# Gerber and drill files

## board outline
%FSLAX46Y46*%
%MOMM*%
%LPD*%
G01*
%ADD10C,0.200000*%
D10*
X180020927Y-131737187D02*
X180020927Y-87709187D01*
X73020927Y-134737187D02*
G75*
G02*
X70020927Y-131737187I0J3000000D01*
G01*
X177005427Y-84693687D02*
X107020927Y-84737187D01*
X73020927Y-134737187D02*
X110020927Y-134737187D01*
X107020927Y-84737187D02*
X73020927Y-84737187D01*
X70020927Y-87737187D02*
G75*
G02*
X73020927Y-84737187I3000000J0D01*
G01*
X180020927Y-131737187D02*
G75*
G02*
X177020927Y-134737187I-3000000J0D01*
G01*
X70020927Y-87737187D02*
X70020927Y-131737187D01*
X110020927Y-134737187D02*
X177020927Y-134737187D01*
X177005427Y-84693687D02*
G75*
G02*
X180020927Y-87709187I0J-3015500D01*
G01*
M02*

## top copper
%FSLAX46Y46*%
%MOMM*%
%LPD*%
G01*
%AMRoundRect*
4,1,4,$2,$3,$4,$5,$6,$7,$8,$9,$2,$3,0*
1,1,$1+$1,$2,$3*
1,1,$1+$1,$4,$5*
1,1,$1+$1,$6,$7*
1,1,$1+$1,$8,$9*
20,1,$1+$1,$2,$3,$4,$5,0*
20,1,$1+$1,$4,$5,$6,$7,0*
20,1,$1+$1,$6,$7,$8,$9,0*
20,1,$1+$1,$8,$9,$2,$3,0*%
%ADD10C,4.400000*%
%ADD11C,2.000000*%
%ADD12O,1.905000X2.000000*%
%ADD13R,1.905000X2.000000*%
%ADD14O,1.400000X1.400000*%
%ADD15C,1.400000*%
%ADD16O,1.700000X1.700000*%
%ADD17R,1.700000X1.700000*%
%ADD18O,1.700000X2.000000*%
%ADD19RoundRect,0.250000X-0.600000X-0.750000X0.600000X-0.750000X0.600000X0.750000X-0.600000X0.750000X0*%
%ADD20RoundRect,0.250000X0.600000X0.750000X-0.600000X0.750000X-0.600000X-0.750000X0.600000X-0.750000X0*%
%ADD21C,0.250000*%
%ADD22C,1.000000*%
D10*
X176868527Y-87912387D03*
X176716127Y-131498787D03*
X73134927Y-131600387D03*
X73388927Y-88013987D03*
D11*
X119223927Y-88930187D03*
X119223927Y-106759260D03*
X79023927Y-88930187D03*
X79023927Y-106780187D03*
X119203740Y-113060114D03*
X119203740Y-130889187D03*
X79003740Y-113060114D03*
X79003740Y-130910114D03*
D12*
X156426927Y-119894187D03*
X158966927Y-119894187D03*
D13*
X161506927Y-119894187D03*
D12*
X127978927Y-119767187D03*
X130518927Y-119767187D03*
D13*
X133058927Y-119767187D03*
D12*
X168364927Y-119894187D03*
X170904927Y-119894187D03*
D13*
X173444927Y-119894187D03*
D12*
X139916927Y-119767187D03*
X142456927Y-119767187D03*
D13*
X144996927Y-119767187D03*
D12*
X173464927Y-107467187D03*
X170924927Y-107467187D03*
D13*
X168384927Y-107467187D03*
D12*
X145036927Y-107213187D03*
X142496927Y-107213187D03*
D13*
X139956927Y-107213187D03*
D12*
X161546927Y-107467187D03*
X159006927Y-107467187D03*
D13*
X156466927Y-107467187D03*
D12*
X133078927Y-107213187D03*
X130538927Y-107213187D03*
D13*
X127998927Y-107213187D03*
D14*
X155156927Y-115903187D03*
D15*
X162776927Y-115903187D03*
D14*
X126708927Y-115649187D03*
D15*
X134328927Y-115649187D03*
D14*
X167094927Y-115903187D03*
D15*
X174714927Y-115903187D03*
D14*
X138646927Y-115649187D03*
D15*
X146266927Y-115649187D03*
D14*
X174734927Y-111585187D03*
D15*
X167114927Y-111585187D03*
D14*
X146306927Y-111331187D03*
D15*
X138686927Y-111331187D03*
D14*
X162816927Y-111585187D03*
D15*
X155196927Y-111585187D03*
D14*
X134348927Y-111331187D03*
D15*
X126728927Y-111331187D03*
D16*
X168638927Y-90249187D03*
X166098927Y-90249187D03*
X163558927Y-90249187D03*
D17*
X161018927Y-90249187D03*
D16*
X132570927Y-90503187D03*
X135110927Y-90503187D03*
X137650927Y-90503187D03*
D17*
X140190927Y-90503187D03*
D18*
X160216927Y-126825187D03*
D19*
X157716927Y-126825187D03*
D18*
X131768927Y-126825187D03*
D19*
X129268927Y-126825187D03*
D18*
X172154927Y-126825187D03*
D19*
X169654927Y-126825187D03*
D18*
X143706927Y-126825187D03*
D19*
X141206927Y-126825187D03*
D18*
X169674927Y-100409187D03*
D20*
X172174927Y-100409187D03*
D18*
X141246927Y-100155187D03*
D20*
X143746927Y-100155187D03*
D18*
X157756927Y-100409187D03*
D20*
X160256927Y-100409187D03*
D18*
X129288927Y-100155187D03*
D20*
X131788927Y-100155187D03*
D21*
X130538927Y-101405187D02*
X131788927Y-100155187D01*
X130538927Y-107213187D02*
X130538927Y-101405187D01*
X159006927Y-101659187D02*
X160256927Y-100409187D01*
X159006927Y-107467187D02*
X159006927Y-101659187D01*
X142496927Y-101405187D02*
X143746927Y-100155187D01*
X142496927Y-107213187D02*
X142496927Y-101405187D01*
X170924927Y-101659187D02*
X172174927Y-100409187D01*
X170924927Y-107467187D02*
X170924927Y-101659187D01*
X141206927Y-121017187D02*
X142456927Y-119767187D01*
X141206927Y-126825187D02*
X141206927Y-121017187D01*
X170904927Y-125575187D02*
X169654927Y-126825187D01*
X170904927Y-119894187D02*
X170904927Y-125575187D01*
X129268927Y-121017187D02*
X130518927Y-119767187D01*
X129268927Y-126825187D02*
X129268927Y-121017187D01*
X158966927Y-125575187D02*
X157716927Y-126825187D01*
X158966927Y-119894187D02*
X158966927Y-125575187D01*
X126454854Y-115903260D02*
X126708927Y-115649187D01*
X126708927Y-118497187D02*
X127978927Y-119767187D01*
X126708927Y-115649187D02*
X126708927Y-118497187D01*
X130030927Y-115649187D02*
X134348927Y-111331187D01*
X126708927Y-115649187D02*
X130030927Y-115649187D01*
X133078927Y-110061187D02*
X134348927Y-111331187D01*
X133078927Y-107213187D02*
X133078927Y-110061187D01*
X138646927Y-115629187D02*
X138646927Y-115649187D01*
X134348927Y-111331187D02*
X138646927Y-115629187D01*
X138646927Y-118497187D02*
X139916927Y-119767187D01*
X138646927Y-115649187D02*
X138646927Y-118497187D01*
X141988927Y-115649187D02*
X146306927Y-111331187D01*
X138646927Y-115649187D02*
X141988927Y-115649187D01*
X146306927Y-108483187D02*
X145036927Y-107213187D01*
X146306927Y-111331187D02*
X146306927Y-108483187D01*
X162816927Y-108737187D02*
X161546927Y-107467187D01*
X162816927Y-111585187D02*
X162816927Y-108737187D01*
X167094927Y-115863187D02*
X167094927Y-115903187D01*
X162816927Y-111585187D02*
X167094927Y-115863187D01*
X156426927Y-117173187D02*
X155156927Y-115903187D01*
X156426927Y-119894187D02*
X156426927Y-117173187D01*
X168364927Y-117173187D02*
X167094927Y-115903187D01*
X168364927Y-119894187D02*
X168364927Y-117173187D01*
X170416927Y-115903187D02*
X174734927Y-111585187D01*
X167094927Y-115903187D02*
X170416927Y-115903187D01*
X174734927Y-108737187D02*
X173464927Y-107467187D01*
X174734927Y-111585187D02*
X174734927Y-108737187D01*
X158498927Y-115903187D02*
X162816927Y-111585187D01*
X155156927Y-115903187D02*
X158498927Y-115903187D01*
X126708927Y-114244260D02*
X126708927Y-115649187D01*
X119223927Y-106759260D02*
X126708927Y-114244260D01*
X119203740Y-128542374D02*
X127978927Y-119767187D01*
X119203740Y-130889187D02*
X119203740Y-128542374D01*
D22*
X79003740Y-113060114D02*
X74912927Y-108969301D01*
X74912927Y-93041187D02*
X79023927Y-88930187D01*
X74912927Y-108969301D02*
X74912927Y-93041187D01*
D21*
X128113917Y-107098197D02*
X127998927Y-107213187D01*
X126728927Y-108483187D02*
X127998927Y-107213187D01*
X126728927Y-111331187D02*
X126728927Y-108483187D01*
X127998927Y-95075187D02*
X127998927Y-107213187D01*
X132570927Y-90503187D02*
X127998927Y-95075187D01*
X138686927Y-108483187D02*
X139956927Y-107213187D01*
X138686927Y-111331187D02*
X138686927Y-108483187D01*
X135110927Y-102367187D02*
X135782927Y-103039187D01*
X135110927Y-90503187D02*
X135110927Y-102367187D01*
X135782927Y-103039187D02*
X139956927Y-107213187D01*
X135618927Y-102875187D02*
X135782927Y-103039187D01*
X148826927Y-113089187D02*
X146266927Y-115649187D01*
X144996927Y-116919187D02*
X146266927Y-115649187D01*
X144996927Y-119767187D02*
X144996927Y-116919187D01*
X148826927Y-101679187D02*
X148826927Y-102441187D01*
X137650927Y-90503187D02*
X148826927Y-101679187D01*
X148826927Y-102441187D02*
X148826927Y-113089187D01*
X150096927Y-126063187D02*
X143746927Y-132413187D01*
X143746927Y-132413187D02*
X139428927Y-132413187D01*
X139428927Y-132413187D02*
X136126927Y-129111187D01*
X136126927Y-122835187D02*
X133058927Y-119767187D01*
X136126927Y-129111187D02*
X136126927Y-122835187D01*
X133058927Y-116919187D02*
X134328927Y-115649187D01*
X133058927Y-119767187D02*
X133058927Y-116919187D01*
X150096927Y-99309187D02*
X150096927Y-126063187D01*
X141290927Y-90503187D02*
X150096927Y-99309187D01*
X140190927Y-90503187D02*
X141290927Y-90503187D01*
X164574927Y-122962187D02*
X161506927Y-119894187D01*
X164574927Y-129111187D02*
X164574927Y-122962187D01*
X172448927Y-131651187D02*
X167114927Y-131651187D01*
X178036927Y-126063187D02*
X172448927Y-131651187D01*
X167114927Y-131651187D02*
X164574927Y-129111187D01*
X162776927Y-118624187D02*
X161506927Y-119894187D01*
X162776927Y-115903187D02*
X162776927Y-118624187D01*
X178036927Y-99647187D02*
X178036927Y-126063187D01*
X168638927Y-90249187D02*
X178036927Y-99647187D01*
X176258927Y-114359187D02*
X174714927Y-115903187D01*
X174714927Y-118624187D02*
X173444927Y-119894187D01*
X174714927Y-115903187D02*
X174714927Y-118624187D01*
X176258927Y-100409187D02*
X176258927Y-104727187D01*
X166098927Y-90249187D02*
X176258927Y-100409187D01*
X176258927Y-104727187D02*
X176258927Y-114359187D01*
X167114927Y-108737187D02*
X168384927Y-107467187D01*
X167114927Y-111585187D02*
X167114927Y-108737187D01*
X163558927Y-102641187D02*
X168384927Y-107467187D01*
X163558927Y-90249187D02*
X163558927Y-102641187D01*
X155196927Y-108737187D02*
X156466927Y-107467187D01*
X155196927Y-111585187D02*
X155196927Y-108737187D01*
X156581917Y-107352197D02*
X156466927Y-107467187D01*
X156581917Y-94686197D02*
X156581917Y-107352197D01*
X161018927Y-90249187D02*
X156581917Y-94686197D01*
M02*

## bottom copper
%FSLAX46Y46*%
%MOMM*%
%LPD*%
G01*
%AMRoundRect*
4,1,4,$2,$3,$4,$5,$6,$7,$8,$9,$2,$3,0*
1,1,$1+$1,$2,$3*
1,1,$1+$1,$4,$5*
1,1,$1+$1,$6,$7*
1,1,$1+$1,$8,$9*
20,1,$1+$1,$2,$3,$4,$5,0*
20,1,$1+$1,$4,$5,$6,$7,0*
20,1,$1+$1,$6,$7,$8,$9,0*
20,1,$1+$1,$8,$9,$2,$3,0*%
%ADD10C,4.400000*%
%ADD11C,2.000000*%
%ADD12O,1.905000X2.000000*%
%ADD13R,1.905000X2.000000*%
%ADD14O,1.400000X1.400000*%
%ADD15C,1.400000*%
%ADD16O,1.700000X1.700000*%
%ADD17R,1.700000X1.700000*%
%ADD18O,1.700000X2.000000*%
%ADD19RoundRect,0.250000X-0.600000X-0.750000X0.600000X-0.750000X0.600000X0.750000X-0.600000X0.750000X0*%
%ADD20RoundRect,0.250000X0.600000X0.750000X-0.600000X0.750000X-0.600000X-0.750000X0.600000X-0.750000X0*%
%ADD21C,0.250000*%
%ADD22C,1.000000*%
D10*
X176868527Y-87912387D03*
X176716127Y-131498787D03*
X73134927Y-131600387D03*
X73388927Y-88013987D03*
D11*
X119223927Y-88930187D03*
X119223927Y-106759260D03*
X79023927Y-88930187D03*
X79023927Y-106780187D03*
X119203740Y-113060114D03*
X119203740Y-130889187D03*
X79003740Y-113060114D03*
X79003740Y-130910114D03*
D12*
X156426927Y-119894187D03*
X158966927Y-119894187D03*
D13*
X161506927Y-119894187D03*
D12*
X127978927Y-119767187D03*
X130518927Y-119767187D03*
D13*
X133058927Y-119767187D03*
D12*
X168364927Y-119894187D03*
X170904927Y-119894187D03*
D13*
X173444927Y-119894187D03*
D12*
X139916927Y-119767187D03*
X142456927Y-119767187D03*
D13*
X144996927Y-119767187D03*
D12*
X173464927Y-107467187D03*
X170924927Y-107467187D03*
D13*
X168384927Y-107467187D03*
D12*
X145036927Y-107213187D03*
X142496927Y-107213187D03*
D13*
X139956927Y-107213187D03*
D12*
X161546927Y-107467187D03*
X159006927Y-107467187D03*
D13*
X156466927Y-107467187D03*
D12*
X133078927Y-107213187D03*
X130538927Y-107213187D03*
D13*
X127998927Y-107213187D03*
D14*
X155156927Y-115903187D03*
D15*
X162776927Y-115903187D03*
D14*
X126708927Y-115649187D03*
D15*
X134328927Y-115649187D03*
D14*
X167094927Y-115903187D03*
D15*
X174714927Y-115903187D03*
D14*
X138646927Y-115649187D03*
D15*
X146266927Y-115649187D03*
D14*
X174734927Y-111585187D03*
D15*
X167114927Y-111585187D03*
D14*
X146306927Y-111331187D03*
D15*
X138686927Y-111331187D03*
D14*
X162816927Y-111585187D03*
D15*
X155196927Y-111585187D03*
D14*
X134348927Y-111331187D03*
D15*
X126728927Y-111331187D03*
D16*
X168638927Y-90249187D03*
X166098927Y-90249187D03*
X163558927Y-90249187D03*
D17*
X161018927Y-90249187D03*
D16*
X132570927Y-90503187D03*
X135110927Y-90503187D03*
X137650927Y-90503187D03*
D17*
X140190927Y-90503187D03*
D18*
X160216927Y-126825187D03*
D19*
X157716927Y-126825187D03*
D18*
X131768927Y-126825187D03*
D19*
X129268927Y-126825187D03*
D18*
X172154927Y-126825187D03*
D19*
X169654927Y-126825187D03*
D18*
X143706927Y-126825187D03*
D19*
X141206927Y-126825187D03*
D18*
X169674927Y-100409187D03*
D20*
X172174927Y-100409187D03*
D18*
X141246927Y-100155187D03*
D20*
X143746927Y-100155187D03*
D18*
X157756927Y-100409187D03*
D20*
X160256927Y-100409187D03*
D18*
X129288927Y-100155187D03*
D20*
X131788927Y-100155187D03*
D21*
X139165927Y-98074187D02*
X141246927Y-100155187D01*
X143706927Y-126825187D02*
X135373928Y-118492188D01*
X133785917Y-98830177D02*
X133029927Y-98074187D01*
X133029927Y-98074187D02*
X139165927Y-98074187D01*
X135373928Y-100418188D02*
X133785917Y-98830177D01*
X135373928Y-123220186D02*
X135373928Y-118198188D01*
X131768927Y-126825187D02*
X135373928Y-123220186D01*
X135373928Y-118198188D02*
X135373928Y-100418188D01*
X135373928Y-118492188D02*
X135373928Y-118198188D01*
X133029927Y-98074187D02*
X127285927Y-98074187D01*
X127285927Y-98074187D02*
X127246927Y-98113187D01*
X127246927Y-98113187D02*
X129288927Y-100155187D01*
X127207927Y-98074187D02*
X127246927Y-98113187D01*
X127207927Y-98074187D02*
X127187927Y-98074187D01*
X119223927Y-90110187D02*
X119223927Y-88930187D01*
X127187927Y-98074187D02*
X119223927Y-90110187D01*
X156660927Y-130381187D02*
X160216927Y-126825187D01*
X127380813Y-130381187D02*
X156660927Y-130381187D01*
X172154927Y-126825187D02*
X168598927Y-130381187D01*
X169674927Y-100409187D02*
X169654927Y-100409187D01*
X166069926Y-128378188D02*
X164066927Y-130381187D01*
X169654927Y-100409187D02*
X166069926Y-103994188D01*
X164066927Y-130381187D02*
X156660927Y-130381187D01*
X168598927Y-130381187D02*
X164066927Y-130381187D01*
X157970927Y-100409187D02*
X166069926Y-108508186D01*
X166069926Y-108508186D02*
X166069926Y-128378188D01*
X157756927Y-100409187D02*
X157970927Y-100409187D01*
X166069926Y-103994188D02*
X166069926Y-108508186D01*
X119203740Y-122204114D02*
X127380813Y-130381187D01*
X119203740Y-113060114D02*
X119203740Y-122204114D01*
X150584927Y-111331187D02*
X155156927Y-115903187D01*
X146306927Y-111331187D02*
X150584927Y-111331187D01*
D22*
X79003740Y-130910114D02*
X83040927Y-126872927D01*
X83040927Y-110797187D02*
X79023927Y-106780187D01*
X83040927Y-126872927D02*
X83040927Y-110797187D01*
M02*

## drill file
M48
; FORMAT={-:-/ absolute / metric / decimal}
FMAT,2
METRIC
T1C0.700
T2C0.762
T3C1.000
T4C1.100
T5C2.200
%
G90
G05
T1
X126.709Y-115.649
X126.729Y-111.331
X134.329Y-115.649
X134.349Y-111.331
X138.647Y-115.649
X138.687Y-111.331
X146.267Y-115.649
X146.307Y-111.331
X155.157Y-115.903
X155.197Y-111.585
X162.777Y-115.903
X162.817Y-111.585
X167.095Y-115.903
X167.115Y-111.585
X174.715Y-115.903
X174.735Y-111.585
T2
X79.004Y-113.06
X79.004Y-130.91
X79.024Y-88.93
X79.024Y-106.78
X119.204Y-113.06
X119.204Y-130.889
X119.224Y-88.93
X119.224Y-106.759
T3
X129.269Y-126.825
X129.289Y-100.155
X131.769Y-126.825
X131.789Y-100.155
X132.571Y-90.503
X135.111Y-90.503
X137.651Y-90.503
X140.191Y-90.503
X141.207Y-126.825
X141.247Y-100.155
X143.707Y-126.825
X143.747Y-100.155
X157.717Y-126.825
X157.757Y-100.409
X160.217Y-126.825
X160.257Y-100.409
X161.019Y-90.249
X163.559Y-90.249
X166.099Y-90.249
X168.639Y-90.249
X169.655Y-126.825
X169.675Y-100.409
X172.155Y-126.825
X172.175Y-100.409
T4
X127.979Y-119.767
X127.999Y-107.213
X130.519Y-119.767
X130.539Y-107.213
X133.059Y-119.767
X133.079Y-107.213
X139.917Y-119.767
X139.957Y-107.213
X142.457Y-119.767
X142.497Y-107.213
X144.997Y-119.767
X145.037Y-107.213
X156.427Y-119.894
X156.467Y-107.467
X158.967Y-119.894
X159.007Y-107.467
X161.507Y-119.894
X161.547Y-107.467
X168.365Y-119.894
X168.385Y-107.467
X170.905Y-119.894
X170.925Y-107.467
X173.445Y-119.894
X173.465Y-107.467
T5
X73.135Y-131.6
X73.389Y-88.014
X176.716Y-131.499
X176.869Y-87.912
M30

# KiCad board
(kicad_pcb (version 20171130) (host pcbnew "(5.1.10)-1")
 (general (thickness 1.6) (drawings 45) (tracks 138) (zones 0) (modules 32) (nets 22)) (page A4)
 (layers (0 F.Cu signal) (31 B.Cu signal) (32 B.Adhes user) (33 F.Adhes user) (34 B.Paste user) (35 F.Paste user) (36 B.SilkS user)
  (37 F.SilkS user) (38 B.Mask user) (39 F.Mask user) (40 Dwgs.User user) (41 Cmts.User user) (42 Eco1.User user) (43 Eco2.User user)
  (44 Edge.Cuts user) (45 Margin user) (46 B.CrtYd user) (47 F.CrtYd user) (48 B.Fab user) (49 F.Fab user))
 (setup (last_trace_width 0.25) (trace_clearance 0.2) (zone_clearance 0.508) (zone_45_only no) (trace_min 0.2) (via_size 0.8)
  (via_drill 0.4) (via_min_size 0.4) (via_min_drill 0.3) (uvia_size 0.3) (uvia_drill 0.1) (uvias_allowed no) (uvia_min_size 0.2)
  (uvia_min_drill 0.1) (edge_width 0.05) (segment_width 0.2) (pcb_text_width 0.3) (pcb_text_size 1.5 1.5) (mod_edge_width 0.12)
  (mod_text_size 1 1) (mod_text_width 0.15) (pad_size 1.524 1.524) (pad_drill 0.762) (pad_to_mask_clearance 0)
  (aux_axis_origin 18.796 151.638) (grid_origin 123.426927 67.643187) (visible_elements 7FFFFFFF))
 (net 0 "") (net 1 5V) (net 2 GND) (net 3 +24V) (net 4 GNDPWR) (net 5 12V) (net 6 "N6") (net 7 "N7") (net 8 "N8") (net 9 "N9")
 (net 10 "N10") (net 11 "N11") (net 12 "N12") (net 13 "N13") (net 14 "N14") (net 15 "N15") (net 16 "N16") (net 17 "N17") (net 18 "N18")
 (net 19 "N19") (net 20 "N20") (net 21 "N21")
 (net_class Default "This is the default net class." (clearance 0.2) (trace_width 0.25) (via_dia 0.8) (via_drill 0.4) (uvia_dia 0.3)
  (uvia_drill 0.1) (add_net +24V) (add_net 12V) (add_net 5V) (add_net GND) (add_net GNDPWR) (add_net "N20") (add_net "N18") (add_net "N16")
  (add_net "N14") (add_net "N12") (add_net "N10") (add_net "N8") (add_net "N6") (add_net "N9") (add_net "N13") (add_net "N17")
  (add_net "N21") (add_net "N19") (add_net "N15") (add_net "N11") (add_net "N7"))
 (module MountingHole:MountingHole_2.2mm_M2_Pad (layer F.Cu) (at 176.868527 87.912387)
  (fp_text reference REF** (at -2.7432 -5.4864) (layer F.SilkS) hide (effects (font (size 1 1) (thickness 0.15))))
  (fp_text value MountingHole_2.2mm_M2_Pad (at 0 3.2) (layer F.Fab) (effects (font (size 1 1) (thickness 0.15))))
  (pad 1 thru_hole circle (at 0 0) (size 4.4 4.4) (drill 2.2) (layers *.Cu *.Mask)))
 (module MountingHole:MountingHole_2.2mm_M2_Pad (layer F.Cu) (at 176.716127 131.498787)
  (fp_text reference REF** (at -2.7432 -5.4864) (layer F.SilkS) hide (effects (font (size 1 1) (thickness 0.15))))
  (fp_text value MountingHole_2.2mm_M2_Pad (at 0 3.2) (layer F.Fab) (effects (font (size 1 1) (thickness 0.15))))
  (pad 1 thru_hole circle (at 0 0) (size 4.4 4.4) (drill 2.2) (layers *.Cu *.Mask)))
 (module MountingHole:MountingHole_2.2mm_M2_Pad (layer F.Cu) (at 73.134927 131.600387)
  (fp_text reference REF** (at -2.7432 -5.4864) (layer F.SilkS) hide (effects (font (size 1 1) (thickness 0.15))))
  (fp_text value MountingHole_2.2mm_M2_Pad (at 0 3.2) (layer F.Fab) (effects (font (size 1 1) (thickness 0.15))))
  (pad 1 thru_hole circle (at 0 0) (size 4.4 4.4) (drill 2.2) (layers *.Cu *.Mask)))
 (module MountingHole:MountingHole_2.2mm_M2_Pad (layer F.Cu) (at 73.388927 88.013987)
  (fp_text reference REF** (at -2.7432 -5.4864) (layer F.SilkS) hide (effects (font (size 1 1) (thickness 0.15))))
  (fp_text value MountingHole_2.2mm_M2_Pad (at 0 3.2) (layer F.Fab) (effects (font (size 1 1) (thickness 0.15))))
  (pad 1 thru_hole circle (at 0 0) (size 4.4 4.4) (drill 2.2) (layers *.Cu *.Mask)))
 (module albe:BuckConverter (layer F.Cu) (at 99.825114 97.86926 270)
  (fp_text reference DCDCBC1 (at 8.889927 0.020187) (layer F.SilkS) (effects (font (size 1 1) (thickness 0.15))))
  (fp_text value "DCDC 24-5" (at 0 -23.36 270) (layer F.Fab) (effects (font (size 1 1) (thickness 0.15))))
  (pad 4 thru_hole circle (at -8.939073 -19.398813 270) (size 2 2) (drill 0.762) (layers *.Cu *.Mask) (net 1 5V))
  (pad 3 thru_hole circle (at 8.89 -19.398813 270) (size 2 2) (drill 0.762) (layers *.Cu *.Mask) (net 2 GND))
  (pad 2 thru_hole circle (at -8.939073 20.801187 270) (size 2 2) (drill 0.762) (layers *.Cu *.Mask) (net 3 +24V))
  (pad 1 thru_hole circle (at 8.910927 20.801187 270) (size 2 2) (drill 0.762) (layers *.Cu *.Mask) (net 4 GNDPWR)))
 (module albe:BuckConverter (layer F.Cu) (at 99.804927 121.999187 270)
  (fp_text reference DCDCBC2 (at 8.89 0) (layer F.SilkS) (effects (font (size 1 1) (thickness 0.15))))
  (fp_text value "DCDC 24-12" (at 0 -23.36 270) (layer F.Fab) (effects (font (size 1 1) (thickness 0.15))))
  (pad 4 thru_hole circle (at -8.939073 -19.398813 270) (size 2 2) (drill 0.762) (layers *.Cu *.Mask) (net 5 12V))
  (pad 3 thru_hole circle (at 8.89 -19.398813 270) (size 2 2) (drill 0.762) (layers *.Cu *.Mask) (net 2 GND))
  (pad 2 thru_hole circle (at -8.939073 20.801187 270) (size 2 2) (drill 0.762) (layers *.Cu *.Mask) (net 3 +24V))
  (pad 1 thru_hole circle (at 8.910927 20.801187 270) (size 2 2) (drill 0.762) (layers *.Cu *.Mask) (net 4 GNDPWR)))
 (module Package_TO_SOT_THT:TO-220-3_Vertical (layer F.Cu) (at 161.506927 119.894187 180)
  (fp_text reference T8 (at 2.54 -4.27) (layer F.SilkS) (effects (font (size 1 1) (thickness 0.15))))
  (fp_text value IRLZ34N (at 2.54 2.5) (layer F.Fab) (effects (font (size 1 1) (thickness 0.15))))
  (pad 3 thru_hole oval (at 5.08 0 180) (size 1.905 2) (drill 1.1) (layers *.Cu *.Mask) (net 2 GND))
  (pad 2 thru_hole oval (at 2.54 0 180) (size 1.905 2) (drill 1.1) (layers *.Cu *.Mask) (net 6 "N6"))
  (pad 1 thru_hole rect (at 0 0 180) (size 1.905 2) (drill 1.1) (layers *.Cu *.Mask) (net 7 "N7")))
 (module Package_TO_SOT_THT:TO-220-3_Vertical (layer F.Cu) (at 133.058927 119.767187 180)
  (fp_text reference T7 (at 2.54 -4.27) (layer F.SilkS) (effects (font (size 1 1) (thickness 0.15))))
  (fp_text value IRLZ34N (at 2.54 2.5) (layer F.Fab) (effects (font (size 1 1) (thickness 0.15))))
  (pad 3 thru_hole oval (at 5.08 0 180) (size 1.905 2) (drill 1.1) (layers *.Cu *.Mask) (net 2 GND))
  (pad 2 thru_hole oval (at 2.54 0 180) (size 1.905 2) (drill 1.1) (layers *.Cu *.Mask) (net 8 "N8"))
  (pad 1 thru_hole rect (at 0 0 180) (size 1.905 2) (drill 1.1) (layers *.Cu *.Mask) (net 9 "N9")))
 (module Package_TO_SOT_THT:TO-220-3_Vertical (layer F.Cu) (at 173.444927 119.894187 180)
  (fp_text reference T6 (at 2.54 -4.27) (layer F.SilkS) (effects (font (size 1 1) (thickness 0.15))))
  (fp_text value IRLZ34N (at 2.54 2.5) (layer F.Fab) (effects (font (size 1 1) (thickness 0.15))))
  (pad 3 thru_hole oval (at 5.08 0 180) (size 1.905 2) (drill 1.1) (layers *.Cu *.Mask) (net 2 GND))
  (pad 2 thru_hole oval (at 2.54 0 180) (size 1.905 2) (drill 1.1) (layers *.Cu *.Mask) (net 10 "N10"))
  (pad 1 thru_hole rect (at 0 0 180) (size 1.905 2) (drill 1.1) (layers *.Cu *.Mask) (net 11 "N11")))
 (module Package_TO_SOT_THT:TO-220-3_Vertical (layer F.Cu) (at 144.996927 119.767187 180)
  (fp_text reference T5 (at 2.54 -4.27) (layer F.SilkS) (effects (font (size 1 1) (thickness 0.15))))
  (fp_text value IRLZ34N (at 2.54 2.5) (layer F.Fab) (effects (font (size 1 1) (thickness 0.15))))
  (pad 3 thru_hole oval (at 5.08 0 180) (size 1.905 2) (drill 1.1) (layers *.Cu *.Mask) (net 2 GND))
  (pad 2 thru_hole oval (at 2.54 0 180) (size 1.905 2) (drill 1.1) (layers *.Cu *.Mask) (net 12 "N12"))
  (pad 1 thru_hole rect (at 0 0 180) (size 1.905 2) (drill 1.1) (layers *.Cu *.Mask) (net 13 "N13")))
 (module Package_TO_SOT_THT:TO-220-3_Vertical (layer F.Cu) (at 168.384927 107.467187)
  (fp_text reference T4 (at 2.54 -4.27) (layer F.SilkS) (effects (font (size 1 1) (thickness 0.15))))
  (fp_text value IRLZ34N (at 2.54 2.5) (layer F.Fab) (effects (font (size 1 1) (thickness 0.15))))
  (pad 3 thru_hole oval (at 5.08 0) (size 1.905 2) (drill 1.1) (layers *.Cu *.Mask) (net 2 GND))
  (pad 2 thru_hole oval (at 2.54 0) (size 1.905 2) (drill 1.1) (layers *.Cu *.Mask) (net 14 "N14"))
  (pad 1 thru_hole rect (at 0 0) (size 1.905 2) (drill 1.1) (layers *.Cu *.Mask) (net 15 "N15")))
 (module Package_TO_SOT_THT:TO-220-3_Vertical (layer F.Cu) (at 139.956927 107.213187)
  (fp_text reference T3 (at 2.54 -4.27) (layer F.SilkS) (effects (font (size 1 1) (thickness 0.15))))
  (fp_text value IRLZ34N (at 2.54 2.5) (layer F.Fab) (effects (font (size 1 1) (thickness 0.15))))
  (pad 3 thru_hole oval (at 5.08 0) (size 1.905 2) (drill 1.1) (layers *.Cu *.Mask) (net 2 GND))
  (pad 2 thru_hole oval (at 2.54 0) (size 1.905 2) (drill 1.1) (layers *.Cu *.Mask) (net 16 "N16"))
  (pad 1 thru_hole rect (at 0 0) (size 1.905 2) (drill 1.1) (layers *.Cu *.Mask) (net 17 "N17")))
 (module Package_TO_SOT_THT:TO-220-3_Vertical (layer F.Cu) (at 156.466927 107.467187)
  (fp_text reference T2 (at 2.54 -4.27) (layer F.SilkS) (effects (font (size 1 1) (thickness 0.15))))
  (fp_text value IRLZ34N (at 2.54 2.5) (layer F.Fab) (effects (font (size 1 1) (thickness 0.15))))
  (pad 3 thru_hole oval (at 5.08 0) (size 1.905 2) (drill 1.1) (layers *.Cu *.Mask) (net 2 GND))
  (pad 2 thru_hole oval (at 2.54 0) (size 1.905 2) (drill 1.1) (layers *.Cu *.Mask) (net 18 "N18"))
  (pad 1 thru_hole rect (at 0 0) (size 1.905 2) (drill 1.1) (layers *.Cu *.Mask) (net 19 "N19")))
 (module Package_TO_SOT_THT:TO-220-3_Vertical (layer F.Cu) (at 127.998927 107.213187)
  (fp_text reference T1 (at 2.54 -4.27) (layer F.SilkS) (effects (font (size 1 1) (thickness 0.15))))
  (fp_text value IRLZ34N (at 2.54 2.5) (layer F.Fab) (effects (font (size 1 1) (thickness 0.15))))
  (pad 3 thru_hole oval (at 5.08 0) (size 1.905 2) (drill 1.1) (layers *.Cu *.Mask) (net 2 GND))
  (pad 2 thru_hole oval (at 2.54 0) (size 1.905 2) (drill 1.1) (layers *.Cu *.Mask) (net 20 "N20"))
  (pad 1 thru_hole rect (at 0 0) (size 1.905 2) (drill 1.1) (layers *.Cu *.Mask) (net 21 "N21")))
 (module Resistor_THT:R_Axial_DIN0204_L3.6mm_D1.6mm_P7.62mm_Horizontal (layer F.Cu) (at 162.776927 115.903187 180)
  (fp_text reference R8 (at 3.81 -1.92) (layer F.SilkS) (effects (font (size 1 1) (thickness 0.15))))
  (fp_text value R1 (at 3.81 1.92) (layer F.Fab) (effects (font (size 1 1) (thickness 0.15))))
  (pad 2 thru_hole oval (at 7.62 0 180) (size 1.4 1.4) (drill 0.7) (layers *.Cu *.Mask) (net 2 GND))
  (pad 1 thru_hole circle (at 0 0 180) (size 1.4 1.4) (drill 0.7) (layers *.Cu *.Mask) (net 7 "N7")))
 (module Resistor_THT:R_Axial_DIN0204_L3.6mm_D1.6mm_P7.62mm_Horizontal (layer F.Cu) (at 134.328927 115.649187 180)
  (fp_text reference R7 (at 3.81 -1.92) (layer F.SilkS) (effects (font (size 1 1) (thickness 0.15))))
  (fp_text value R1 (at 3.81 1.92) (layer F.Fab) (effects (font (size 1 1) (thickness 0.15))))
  (pad 2 thru_hole oval (at 7.62 0 180) (size 1.4 1.4) (drill 0.7) (layers *.Cu *.Mask) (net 2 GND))
  (pad 1 thru_hole circle (at 0 0 180) (size 1.4 1.4) (drill 0.7) (layers *.Cu *.Mask) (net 9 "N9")))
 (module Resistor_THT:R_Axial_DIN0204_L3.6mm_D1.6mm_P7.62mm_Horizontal (layer F.Cu) (at 174.714927 115.903187 180)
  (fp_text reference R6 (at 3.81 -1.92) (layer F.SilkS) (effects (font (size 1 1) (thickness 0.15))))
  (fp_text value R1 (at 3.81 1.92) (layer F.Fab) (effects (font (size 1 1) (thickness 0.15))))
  (pad 2 thru_hole oval (at 7.62 0 180) (size 1.4 1.4) (drill 0.7) (layers *.Cu *.Mask) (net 2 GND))
  (pad 1 thru_hole circle (at 0 0 180) (size 1.4 1.4) (drill 0.7) (layers *.Cu *.Mask) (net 11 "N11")))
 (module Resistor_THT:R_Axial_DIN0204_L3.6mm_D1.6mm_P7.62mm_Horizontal (layer F.Cu) (at 146.266927 115.649187 180)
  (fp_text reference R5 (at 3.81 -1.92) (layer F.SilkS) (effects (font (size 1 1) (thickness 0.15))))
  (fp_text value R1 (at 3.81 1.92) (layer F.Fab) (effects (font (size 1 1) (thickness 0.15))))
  (pad 2 thru_hole oval (at 7.62 0 180) (size 1.4 1.4) (drill 0.7) (layers *.Cu *.Mask) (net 2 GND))
  (pad 1 thru_hole circle (at 0 0 180) (size 1.4 1.4) (drill 0.7) (layers *.Cu *.Mask) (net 13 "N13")))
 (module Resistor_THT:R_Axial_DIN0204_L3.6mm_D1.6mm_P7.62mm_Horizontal (layer F.Cu) (at 167.114927 111.585187)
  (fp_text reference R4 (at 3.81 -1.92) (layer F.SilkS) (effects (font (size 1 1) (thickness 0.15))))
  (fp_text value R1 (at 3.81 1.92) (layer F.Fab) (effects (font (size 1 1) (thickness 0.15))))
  (pad 2 thru_hole oval (at 7.62 0) (size 1.4 1.4) (drill 0.7) (layers *.Cu *.Mask) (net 2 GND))
  (pad 1 thru_hole circle (at 0 0) (size 1.4 1.4) (drill 0.7) (layers *.Cu *.Mask) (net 15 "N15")))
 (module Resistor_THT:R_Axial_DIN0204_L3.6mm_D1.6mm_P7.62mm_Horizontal (layer F.Cu) (at 138.686927 111.331187)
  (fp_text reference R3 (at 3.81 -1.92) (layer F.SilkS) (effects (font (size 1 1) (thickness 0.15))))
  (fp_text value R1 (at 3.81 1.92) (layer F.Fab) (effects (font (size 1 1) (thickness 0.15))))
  (pad 2 thru_hole oval (at 7.62 0) (size 1.4 1.4) (drill 0.7) (layers *.Cu *.Mask) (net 2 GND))
  (pad 1 thru_hole circle (at 0 0) (size 1.4 1.4) (drill 0.7) (layers *.Cu *.Mask) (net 17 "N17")))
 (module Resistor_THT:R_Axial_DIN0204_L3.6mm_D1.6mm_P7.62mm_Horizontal (layer F.Cu) (at 155.196927 111.585187)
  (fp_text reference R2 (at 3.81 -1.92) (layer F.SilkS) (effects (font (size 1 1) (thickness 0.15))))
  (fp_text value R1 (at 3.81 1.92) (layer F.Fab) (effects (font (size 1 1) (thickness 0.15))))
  (pad 2 thru_hole oval (at 7.62 0) (size 1.4 1.4) (drill 0.7) (layers *.Cu *.Mask) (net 2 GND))
  (pad 1 thru_hole circle (at 0 0) (size 1.4 1.4) (drill 0.7) (layers *.Cu *.Mask) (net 19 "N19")))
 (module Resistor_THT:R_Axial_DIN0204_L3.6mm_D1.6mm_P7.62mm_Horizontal (layer F.Cu) (at 126.728927 111.331187)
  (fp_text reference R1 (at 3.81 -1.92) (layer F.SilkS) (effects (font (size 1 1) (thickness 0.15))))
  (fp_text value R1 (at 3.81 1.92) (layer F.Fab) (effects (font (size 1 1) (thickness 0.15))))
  (pad 2 thru_hole oval (at 7.62 0) (size 1.4 1.4) (drill 0.7) (layers *.Cu *.Mask) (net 2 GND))
  (pad 1 thru_hole circle (at 0 0) (size 1.4 1.4) (drill 0.7) (layers *.Cu *.Mask) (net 21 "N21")))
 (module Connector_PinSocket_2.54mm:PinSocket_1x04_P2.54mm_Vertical (layer F.Cu) (at 161.018927 90.249187 90)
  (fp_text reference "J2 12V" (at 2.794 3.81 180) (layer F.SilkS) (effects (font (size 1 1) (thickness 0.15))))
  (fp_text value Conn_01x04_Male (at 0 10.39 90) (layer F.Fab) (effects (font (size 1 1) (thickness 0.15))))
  (pad 4 thru_hole oval (at 0 7.62 90) (size 1.7 1.7) (drill 1) (layers *.Cu *.Mask) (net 7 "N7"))
  (pad 3 thru_hole oval (at 0 5.08 90) (size 1.7 1.7) (drill 1) (layers *.Cu *.Mask) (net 11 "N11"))
  (pad 2 thru_hole oval (at 0 2.54 90) (size 1.7 1.7) (drill 1) (layers *.Cu *.Mask) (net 15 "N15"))
  (pad 1 thru_hole rect (at 0 0 90) (size 1.7 1.7) (drill 1) (layers *.Cu *.Mask) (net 19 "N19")))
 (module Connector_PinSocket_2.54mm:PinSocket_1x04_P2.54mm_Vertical (layer F.Cu) (at 140.190927 90.503187 270)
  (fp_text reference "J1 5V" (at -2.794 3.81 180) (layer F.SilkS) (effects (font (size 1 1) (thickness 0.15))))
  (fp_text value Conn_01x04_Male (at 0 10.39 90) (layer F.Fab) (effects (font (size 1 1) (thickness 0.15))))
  (pad 4 thru_hole oval (at 0 7.62 270) (size 1.7 1.7) (drill 1) (layers *.Cu *.Mask) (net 21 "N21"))
  (pad 3 thru_hole oval (at 0 5.08 270) (size 1.7 1.7) (drill 1) (layers *.Cu *.Mask) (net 17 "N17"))
  (pad 2 thru_hole oval (at 0 2.54 270) (size 1.7 1.7) (drill 1) (layers *.Cu *.Mask) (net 13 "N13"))
  (pad 1 thru_hole rect (at 0 0 270) (size 1.7 1.7) (drill 1) (layers *.Cu *.Mask) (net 9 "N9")))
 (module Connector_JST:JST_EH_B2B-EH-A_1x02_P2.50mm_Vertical (layer F.Cu) (at 157.716927 126.825187)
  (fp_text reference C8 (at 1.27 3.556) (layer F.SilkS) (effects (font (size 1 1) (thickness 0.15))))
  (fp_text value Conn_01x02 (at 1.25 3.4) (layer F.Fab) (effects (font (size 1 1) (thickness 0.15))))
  (pad 2 thru_hole oval (at 2.5 0) (size 1.7 2) (drill 1) (layers *.Cu *.Mask) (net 5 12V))
  (pad 1 thru_hole roundrect (at 0 0) (size 1.7 2) (drill 1) (layers *.Cu *.Mask) (roundrect_rratio 0.147059) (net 6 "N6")))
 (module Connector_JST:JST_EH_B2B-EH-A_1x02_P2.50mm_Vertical (layer F.Cu) (at 129.268927 126.825187)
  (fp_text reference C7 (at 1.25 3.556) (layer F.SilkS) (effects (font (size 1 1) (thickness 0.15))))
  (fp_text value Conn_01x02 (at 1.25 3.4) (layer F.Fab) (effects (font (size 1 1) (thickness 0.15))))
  (pad 2 thru_hole oval (at 2.5 0) (size 1.7 2) (drill 1) (layers *.Cu *.Mask) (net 1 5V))
  (pad 1 thru_hole roundrect (at 0 0) (size 1.7 2) (drill 1) (layers *.Cu *.Mask) (roundrect_rratio 0.147059) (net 8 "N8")))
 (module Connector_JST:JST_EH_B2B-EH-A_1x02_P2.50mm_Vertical (layer F.Cu) (at 169.654927 126.825187)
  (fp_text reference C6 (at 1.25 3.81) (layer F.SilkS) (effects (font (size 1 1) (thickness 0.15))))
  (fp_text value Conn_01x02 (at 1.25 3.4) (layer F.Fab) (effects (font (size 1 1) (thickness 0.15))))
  (pad 2 thru_hole oval (at 2.5 0) (size 1.7 2) (drill 1) (layers *.Cu *.Mask) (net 5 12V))
  (pad 1 thru_hole roundrect (at 0 0) (size 1.7 2) (drill 1) (layers *.Cu *.Mask) (roundrect_rratio 0.147059) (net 10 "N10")))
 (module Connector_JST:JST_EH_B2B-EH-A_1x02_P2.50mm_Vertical (layer F.Cu) (at 141.206927 126.825187)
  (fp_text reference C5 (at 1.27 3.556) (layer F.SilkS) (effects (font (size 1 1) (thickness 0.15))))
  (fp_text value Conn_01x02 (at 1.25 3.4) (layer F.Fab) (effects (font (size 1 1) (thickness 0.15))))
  (pad 2 thru_hole oval (at 2.5 0) (size 1.7 2) (drill 1) (layers *.Cu *.Mask) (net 1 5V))
  (pad 1 thru_hole roundrect (at 0 0) (size 1.7 2) (drill 1) (layers *.Cu *.Mask) (roundrect_rratio 0.147059) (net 12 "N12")))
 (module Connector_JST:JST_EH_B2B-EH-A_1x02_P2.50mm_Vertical (layer F.Cu) (at 172.174927 100.409187 180)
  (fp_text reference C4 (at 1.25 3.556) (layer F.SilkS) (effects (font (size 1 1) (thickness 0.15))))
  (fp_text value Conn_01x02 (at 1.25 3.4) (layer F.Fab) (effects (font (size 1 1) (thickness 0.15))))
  (pad 2 thru_hole oval (at 2.5 0 180) (size 1.7 2) (drill 1) (layers *.Cu *.Mask) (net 5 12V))
  (pad 1 thru_hole roundrect (at 0 0 180) (size 1.7 2) (drill 1) (layers *.Cu *.Mask) (roundrect_rratio 0.147059) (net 14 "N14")))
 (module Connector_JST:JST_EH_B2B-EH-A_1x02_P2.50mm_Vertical (layer F.Cu) (at 143.746927 100.155187 180)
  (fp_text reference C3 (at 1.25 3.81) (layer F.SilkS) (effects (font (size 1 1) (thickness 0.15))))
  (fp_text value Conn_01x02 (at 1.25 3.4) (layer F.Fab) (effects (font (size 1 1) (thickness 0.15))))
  (pad 2 thru_hole oval (at 2.5 0 180) (size 1.7 2) (drill 1) (layers *.Cu *.Mask) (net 1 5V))
  (pad 1 thru_hole roundrect (at 0 0 180) (size 1.7 2) (drill 1) (layers *.Cu *.Mask) (roundrect_rratio 0.147059) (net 16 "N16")))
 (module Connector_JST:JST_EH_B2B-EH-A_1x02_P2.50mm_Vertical (layer F.Cu) (at 160.256927 100.409187 180)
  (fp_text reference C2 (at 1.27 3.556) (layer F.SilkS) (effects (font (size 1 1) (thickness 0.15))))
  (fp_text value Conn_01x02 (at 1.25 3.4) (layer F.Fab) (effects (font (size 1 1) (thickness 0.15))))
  (pad 2 thru_hole oval (at 2.5 0 180) (size 1.7 2) (drill 1) (layers *.Cu *.Mask) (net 5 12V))
  (pad 1 thru_hole roundrect (at 0 0 180) (size 1.7 2) (drill 1) (layers *.Cu *.Mask) (roundrect_rratio 0.147059) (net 18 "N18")))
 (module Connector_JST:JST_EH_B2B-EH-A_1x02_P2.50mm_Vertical (layer F.Cu) (at 131.788927 100.155187 180)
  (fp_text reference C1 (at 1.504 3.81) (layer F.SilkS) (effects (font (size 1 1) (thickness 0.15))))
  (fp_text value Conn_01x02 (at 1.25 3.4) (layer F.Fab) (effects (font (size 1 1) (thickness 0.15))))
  (pad 2 thru_hole oval (at 2.5 0 180) (size 1.7 2) (drill 1) (layers *.Cu *.Mask) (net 1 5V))
  (pad 1 thru_hole roundrect (at 0 0 180) (size 1.7 2) (drill 1) (layers *.Cu *.Mask) (roundrect_rratio 0.147059) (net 20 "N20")))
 (gr_line (start 180.020927 131.737187) (end 180.020927 87.709187) (layer Edge.Cuts) (width 0.2))
 (gr_arc (start 73.020927 131.737187) (end 70.020927 131.737187) (angle -90) (layer Edge.Cuts) (width 0.2))
 (gr_line (start 177.005427 84.693687) (end 107.020927 84.737187) (layer Edge.Cuts) (width 0.2))
 (gr_line (start 73.020927 134.737187) (end 110.020927 134.737187) (layer Edge.Cuts) (width 0.2))
 (gr_line (start 107.020927 84.737187) (end 73.020927 84.737187) (layer Edge.Cuts) (width 0.2))
 (gr_arc (start 73.020927 87.737187) (end 73.020927 84.737187) (angle -90) (layer Edge.Cuts) (width 0.2))
 (gr_arc (start 177.020927 131.737187) (end 177.020927 134.737187) (angle -90) (layer Edge.Cuts) (width 0.2))
 (gr_line (start 70.020927 87.737187) (end 70.020927 131.737187) (layer Edge.Cuts) (width 0.2))
 (gr_line (start 110.020927 134.737187) (end 177.020927 134.737187) (layer Edge.Cuts) (width 0.2))
 (gr_arc (start 177.005427 87.709187) (end 180.020927 87.709187) (angle -90) (layer Edge.Cuts) (width 0.2))
 (segment (start 139.165927 98.074187) (end 141.246927 100.155187) (width 0.25) (layer B.Cu) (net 1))
 (segment (start 143.706927 126.825187) (end 135.373928 118.492188) (width 0.25) (layer B.Cu) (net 1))
 (segment (start 133.785917 98.830177) (end 133.029927 98.074187) (width 0.25) (layer B.Cu) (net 1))
 (segment (start 133.029927 98.074187) (end 139.165927 98.074187) (width 0.25) (layer B.Cu) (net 1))
 (segment (start 135.373928 100.418188) (end 133.785917 98.830177) (width 0.25) (layer B.Cu) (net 1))
 (segment (start 135.373928 123.220186) (end 135.373928 118.198188) (width 0.25) (layer B.Cu) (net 1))
 (segment (start 131.768927 126.825187) (end 135.373928 123.220186) (width 0.25) (layer B.Cu) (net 1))
 (segment (start 135.373928 118.198188) (end 135.373928 100.418188) (width 0.25) (layer B.Cu) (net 1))
 (segment (start 135.373928 118.492188) (end 135.373928 118.198188) (width 0.25) (layer B.Cu) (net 1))
 (segment (start 133.029927 98.074187) (end 127.285927 98.074187) (width 0.25) (layer B.Cu) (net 1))
 (segment (start 127.285927 98.074187) (end 127.246927 98.113187) (width 0.25) (layer B.Cu) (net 1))
 (segment (start 127.246927 98.113187) (end 129.288927 100.155187) (width 0.25) (layer B.Cu) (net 1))
 (segment (start 127.207927 98.074187) (end 127.246927 98.113187) (width 0.25) (layer B.Cu) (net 1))
 (segment (start 127.207927 98.074187) (end 127.187927 98.074187) (width 0.25) (layer B.Cu) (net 1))
 (segment (start 119.223927 90.110187) (end 119.223927 88.930187) (width 0.25) (layer B.Cu) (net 1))
 (segment (start 127.187927 98.074187) (end 119.223927 90.110187) (width 0.25) (layer B.Cu) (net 1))
 (segment (start 130.538927 101.405187) (end 131.788927 100.155187) (width 0.25) (layer F.Cu) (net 20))
 (segment (start 130.538927 107.213187) (end 130.538927 101.405187) (width 0.25) (layer F.Cu) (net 20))
 (segment (start 156.660927 130.381187) (end 160.216927 126.825187) (width 0.25) (layer B.Cu) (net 5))
 (segment (start 127.380813 130.381187) (end 156.660927 130.381187) (width 0.25) (layer B.Cu) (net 5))
 (segment (start 172.154927 126.825187) (end 168.598927 130.381187) (width 0.25) (layer B.Cu) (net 5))
 (segment (start 169.674927 100.409187) (end 169.654927 100.409187) (width 0.25) (layer B.Cu) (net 5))
 (segment (start 166.069926 128.378188) (end 164.066927 130.381187) (width 0.25) (layer B.Cu) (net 5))
 (segment (start 169.654927 100.409187) (end 166.069926 103.994188) (width 0.25) (layer B.Cu) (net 5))
 (segment (start 164.066927 130.381187) (end 156.660927 130.381187) (width 0.25) (layer B.Cu) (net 5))
 (segment (start 168.598927 130.381187) (end 164.066927 130.381187) (width 0.25) (layer B.Cu) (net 5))
 (segment (start 157.970927 100.409187) (end 166.069926 108.508186) (width 0.25) (layer B.Cu) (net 5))
 (segment (start 166.069926 108.508186) (end 166.069926 128.378188) (width 0.25) (layer B.Cu) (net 5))
 (segment (start 157.756927 100.409187) (end 157.970927 100.409187) (width 0.25) (layer B.Cu) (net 5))
 (segment (start 166.069926 103.994188) (end 166.069926 108.508186) (width 0.25) (layer B.Cu) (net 5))
 (segment (start 119.20374 122.204114) (end 127.380813 130.381187) (width 0.25) (layer B.Cu) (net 5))
 (segment (start 119.20374 113.060114) (end 119.20374 122.204114) (width 0.25) (layer B.Cu) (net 5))
 (segment (start 159.006927 101.659187) (end 160.256927 100.409187) (width 0.25) (layer F.Cu) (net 18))
 (segment (start 159.006927 107.467187) (end 159.006927 101.659187) (width 0.25) (layer F.Cu) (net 18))
 (segment (start 142.496927 101.405187) (end 143.746927 100.155187) (width 0.25) (layer F.Cu) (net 16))
 (segment (start 142.496927 107.213187) (end 142.496927 101.405187) (width 0.25) (layer F.Cu) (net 16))
 (segment (start 170.924927 101.659187) (end 172.174927 100.409187) (width 0.25) (layer F.Cu) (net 14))
 (segment (start 170.924927 107.467187) (end 170.924927 101.659187) (width 0.25) (layer F.Cu) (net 14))
 (segment (start 141.206927 121.017187) (end 142.456927 119.767187) (width 0.25) (layer F.Cu) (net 12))
 (segment (start 141.206927 126.825187) (end 141.206927 121.017187) (width 0.25) (layer F.Cu) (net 12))
 (segment (start 170.904927 125.575187) (end 169.654927 126.825187) (width 0.25) (layer F.Cu) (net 10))
 (segment (start 170.904927 119.894187) (end 170.904927 125.575187) (width 0.25) (layer F.Cu) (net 10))
 (segment (start 129.268927 121.017187) (end 130.518927 119.767187) (width 0.25) (layer F.Cu) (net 8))
 (segment (start 129.268927 126.825187) (end 129.268927 121.017187) (width 0.25) (layer F.Cu) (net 8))
 (segment (start 158.966927 125.575187) (end 157.716927 126.825187) (width 0.25) (layer F.Cu) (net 6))
 (segment (start 158.966927 119.894187) (end 158.966927 125.575187) (width 0.25) (layer F.Cu) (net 6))
 (segment (start 126.454854 115.90326) (end 126.708927 115.649187) (width 0.25) (layer F.Cu) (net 2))
 (segment (start 126.708927 118.497187) (end 127.978927 119.767187) (width 0.25) (layer F.Cu) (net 2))
 (segment (start 126.708927 115.649187) (end 126.708927 118.497187) (width 0.25) (layer F.Cu) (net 2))
 (segment (start 130.030927 115.649187) (end 134.348927 111.331187) (width 0.25) (layer F.Cu) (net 2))
 (segment (start 126.708927 115.649187) (end 130.030927 115.649187) (width 0.25) (layer F.Cu) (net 2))
 (segment (start 133.078927 110.061187) (end 134.348927 111.331187) (width 0.25) (layer F.Cu) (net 2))
 (segment (start 133.078927 107.213187) (end 133.078927 110.061187) (width 0.25) (layer F.Cu) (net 2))
 (segment (start 138.646927 115.629187) (end 138.646927 115.649187) (width 0.25) (layer F.Cu) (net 2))
 (segment (start 134.348927 111.331187) (end 138.646927 115.629187) (width 0.25) (layer F.Cu) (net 2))
 (segment (start 138.646927 118.497187) (end 139.916927 119.767187) (width 0.25) (layer F.Cu) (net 2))
 (segment (start 138.646927 115.649187) (end 138.646927 118.497187) (width 0.25) (layer F.Cu) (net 2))
 (segment (start 141.988927 115.649187) (end 146.306927 111.331187) (width 0.25) (layer F.Cu) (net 2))
 (segment (start 138.646927 115.649187) (end 141.988927 115.649187) (width 0.25) (layer F.Cu) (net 2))
 (segment (start 146.306927 108.483187) (end 145.036927 107.213187) (width 0.25) (layer F.Cu) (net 2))
 (segment (start 146.306927 111.331187) (end 146.306927 108.483187) (width 0.25) (layer F.Cu) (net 2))
 (segment (start 162.816927 108.737187) (end 161.546927 107.467187) (width 0.25) (layer F.Cu) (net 2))
 (segment (start 162.816927 111.585187) (end 162.816927 108.737187) (width 0.25) (layer F.Cu) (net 2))
 (segment (start 167.094927 115.863187) (end 167.094927 115.903187) (width 0.25) (layer F.Cu) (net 2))
 (segment (start 162.816927 111.585187) (end 167.094927 115.863187) (width 0.25) (layer F.Cu) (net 2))
 (segment (start 156.426927 117.173187) (end 155.156927 115.903187) (width 0.25) (layer F.Cu) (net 2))
 (segment (start 156.426927 119.894187) (end 156.426927 117.173187) (width 0.25) (layer F.Cu) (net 2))
 (segment (start 168.364927 117.173187) (end 167.094927 115.903187) (width 0.25) (layer F.Cu) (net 2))
 (segment (start 168.364927 119.894187) (end 168.364927 117.173187) (width 0.25) (layer F.Cu) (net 2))
 (segment (start 170.416927 115.903187) (end 174.734927 111.585187) (width 0.25) (layer F.Cu) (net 2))
 (segment (start 167.094927 115.903187) (end 170.416927 115.903187) (width 0.25) (layer F.Cu) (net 2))
 (segment (start 174.734927 108.737187) (end 173.464927 107.467187) (width 0.25) (layer F.Cu) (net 2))
 (segment (start 174.734927 111.585187) (end 174.734927 108.737187) (width 0.25) (layer F.Cu) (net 2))
 (segment (start 158.498927 115.903187) (end 162.816927 111.585187) (width 0.25) (layer F.Cu) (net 2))
 (segment (start 155.156927 115.903187) (end 158.498927 115.903187) (width 0.25) (layer F.Cu) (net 2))
 (segment (start 150.584927 111.331187) (end 155.156927 115.903187) (width 0.25) (layer B.Cu) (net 2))
 (segment (start 146.306927 111.331187) (end 150.584927 111.331187) (width 0.25) (layer B.Cu) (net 2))
 (segment (start 126.708927 114.24426) (end 126.708927 115.649187) (width 0.25) (layer F.Cu) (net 2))
 (segment (start 119.223927 106.75926) (end 126.708927 114.24426) (width 0.25) (layer F.Cu) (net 2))
 (segment (start 119.20374 128.542374) (end 127.978927 119.767187) (width 0.25) (layer F.Cu) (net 2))
 (segment (start 119.20374 130.889187) (end 119.20374 128.542374) (width 0.25) (layer F.Cu) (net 2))
 (segment (start 79.00374 113.060114) (end 74.912927 108.969301) (width 1) (layer F.Cu) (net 3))
 (segment (start 74.912927 93.041187) (end 79.023927 88.930187) (width 1) (layer F.Cu) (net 3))
 (segment (start 74.912927 108.969301) (end 74.912927 93.041187) (width 1) (layer F.Cu) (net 3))
 (segment (start 79.00374 130.910114) (end 83.040927 126.872927) (width 1) (layer B.Cu) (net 4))
 (segment (start 83.040927 110.797187) (end 79.023927 106.780187) (width 1) (layer B.Cu) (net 4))
 (segment (start 83.040927 126.872927) (end 83.040927 110.797187) (width 1) (layer B.Cu) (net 4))
 (segment (start 128.113917 107.098197) (end 127.998927 107.213187) (width 0.25) (layer F.Cu) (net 21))
 (segment (start 126.728927 108.483187) (end 127.998927 107.213187) (width 0.25) (layer F.Cu) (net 21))
 (segment (start 126.728927 111.331187) (end 126.728927 108.483187) (width 0.25) (layer F.Cu) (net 21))
 (segment (start 127.998927 95.075187) (end 127.998927 107.213187) (width 0.25) (layer F.Cu) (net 21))
 (segment (start 132.570927 90.503187) (end 127.998927 95.075187) (width 0.25) (layer F.Cu) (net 21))
 (segment (start 138.686927 108.483187) (end 139.956927 107.213187) (width 0.25) (layer F.Cu) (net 17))
 (segment (start 138.686927 111.331187) (end 138.686927 108.483187) (width 0.25) (layer F.Cu) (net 17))
 (segment (start 135.110927 102.367187) (end 135.782927 103.039187) (width 0.25) (layer F.Cu) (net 17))
 (segment (start 135.110927 90.503187) (end 135.110927 102.367187) (width 0.25) (layer F.Cu) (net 17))
 (segment (start 135.782927 103.039187) (end 139.956927 107.213187) (width 0.25) (layer F.Cu) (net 17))
 (segment (start 135.618927 102.875187) (end 135.782927 103.039187) (width 0.25) (layer F.Cu) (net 17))
 (segment (start 148.826927 113.089187) (end 146.266927 115.649187) (width 0.25) (layer F.Cu) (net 13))
 (segment (start 144.996927 116.919187) (end 146.266927 115.649187) (width 0.25) (layer F.Cu) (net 13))
 (segment (start 144.996927 119.767187) (end 144.996927 116.919187) (width 0.25) (layer F.Cu) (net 13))
 (segment (start 148.826927 101.679187) (end 148.826927 102.441187) (width 0.25) (layer F.Cu) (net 13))
 (segment (start 137.650927 90.503187) (end 148.826927 101.679187) (width 0.25) (layer F.Cu) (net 13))
 (segment (start 148.826927 102.441187) (end 148.826927 113.089187) (width 0.25) (layer F.Cu) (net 13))
 (segment (start 150.096927 126.063187) (end 143.746927 132.413187) (width 0.25) (layer F.Cu) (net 9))
 (segment (start 143.746927 132.413187) (end 139.428927 132.413187) (width 0.25) (layer F.Cu) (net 9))
 (segment (start 139.428927 132.413187) (end 136.126927 129.111187) (width 0.25) (layer F.Cu) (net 9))
 (segment (start 136.126927 122.835187) (end 133.058927 119.767187) (width 0.25) (layer F.Cu) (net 9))
 (segment (start 136.126927 129.111187) (end 136.126927 122.835187) (width 0.25) (layer F.Cu) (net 9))
 (segment (start 133.058927 116.919187) (end 134.328927 115.649187) (width 0.25) (layer F.Cu) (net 9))
 (segment (start 133.058927 119.767187) (end 133.058927 116.919187) (width 0.25) (layer F.Cu) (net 9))
 (segment (start 150.096927 99.309187) (end 150.096927 126.063187) (width 0.25) (layer F.Cu) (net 9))
 (segment (start 141.290927 90.503187) (end 150.096927 99.309187) (width 0.25) (layer F.Cu) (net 9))
 (segment (start 140.190927 90.503187) (end 141.290927 90.503187) (width 0.25) (layer F.Cu) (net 9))
 (segment (start 164.574927 122.962187) (end 161.506927 119.894187) (width 0.25) (layer F.Cu) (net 7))
 (segment (start 164.574927 129.111187) (end 164.574927 122.962187) (width 0.25) (layer F.Cu) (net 7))
 (segment (start 172.448927 131.651187) (end 167.114927 131.651187) (width 0.25) (layer F.Cu) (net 7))
 (segment (start 178.036927 126.063187) (end 172.448927 131.651187) (width 0.25) (layer F.Cu) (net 7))
 (segment (start 167.114927 131.651187) (end 164.574927 129.111187) (width 0.25) (layer F.Cu) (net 7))
 (segment (start 162.776927 118.624187) (end 161.506927 119.894187) (width 0.25) (layer F.Cu) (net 7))
 (segment (start 162.776927 115.903187) (end 162.776927 118.624187) (width 0.25) (layer F.Cu) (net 7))
 (segment (start 178.036927 99.647187) (end 178.036927 126.063187) (width 0.25) (layer F.Cu) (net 7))
 (segment (start 168.638927 90.249187) (end 178.036927 99.647187) (width 0.25) (layer F.Cu) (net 7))
 (segment (start 176.258927 114.359187) (end 174.714927 115.903187) (width 0.25) (layer F.Cu) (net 11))
 (segment (start 174.714927 118.624187) (end 173.444927 119.894187) (width 0.25) (layer F.Cu) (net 11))
 (segment (start 174.714927 115.903187) (end 174.714927 118.624187) (width 0.25) (layer F.Cu) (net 11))
 (segment (start 176.258927 100.409187) (end 176.258927 104.727187) (width 0.25) (layer F.Cu) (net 11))
 (segment (start 166.098927 90.249187) (end 176.258927 100.409187) (width 0.25) (layer F.Cu) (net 11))
 (segment (start 176.258927 104.727187) (end 176.258927 114.359187) (width 0.25) (layer F.Cu) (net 11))
 (segment (start 167.114927 108.737187) (end 168.384927 107.467187) (width 0.25) (layer F.Cu) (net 15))
 (segment (start 167.114927 111.585187) (end 167.114927 108.737187) (width 0.25) (layer F.Cu) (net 15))
 (segment (start 163.558927 102.641187) (end 168.384927 107.467187) (width 0.25) (layer F.Cu) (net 15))
 (segment (start 163.558927 90.249187) (end 163.558927 102.641187) (width 0.25) (layer F.Cu) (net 15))
 (segment (start 155.196927 108.737187) (end 156.466927 107.467187) (width 0.25) (layer F.Cu) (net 19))
 (segment (start 155.196927 111.585187) (end 155.196927 108.737187) (width 0.25) (layer F.Cu) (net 19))
 (segment (start 156.581917 107.352197) (end 156.466927 107.467187) (width 0.25) (layer F.Cu) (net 19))
 (segment (start 156.581917 94.686197) (end 156.581917 107.352197) (width 0.25) (layer F.Cu) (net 19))
 (segment (start 161.018927 90.249187) (end 156.581917 94.686197) (width 0.25) (layer F.Cu) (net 19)))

